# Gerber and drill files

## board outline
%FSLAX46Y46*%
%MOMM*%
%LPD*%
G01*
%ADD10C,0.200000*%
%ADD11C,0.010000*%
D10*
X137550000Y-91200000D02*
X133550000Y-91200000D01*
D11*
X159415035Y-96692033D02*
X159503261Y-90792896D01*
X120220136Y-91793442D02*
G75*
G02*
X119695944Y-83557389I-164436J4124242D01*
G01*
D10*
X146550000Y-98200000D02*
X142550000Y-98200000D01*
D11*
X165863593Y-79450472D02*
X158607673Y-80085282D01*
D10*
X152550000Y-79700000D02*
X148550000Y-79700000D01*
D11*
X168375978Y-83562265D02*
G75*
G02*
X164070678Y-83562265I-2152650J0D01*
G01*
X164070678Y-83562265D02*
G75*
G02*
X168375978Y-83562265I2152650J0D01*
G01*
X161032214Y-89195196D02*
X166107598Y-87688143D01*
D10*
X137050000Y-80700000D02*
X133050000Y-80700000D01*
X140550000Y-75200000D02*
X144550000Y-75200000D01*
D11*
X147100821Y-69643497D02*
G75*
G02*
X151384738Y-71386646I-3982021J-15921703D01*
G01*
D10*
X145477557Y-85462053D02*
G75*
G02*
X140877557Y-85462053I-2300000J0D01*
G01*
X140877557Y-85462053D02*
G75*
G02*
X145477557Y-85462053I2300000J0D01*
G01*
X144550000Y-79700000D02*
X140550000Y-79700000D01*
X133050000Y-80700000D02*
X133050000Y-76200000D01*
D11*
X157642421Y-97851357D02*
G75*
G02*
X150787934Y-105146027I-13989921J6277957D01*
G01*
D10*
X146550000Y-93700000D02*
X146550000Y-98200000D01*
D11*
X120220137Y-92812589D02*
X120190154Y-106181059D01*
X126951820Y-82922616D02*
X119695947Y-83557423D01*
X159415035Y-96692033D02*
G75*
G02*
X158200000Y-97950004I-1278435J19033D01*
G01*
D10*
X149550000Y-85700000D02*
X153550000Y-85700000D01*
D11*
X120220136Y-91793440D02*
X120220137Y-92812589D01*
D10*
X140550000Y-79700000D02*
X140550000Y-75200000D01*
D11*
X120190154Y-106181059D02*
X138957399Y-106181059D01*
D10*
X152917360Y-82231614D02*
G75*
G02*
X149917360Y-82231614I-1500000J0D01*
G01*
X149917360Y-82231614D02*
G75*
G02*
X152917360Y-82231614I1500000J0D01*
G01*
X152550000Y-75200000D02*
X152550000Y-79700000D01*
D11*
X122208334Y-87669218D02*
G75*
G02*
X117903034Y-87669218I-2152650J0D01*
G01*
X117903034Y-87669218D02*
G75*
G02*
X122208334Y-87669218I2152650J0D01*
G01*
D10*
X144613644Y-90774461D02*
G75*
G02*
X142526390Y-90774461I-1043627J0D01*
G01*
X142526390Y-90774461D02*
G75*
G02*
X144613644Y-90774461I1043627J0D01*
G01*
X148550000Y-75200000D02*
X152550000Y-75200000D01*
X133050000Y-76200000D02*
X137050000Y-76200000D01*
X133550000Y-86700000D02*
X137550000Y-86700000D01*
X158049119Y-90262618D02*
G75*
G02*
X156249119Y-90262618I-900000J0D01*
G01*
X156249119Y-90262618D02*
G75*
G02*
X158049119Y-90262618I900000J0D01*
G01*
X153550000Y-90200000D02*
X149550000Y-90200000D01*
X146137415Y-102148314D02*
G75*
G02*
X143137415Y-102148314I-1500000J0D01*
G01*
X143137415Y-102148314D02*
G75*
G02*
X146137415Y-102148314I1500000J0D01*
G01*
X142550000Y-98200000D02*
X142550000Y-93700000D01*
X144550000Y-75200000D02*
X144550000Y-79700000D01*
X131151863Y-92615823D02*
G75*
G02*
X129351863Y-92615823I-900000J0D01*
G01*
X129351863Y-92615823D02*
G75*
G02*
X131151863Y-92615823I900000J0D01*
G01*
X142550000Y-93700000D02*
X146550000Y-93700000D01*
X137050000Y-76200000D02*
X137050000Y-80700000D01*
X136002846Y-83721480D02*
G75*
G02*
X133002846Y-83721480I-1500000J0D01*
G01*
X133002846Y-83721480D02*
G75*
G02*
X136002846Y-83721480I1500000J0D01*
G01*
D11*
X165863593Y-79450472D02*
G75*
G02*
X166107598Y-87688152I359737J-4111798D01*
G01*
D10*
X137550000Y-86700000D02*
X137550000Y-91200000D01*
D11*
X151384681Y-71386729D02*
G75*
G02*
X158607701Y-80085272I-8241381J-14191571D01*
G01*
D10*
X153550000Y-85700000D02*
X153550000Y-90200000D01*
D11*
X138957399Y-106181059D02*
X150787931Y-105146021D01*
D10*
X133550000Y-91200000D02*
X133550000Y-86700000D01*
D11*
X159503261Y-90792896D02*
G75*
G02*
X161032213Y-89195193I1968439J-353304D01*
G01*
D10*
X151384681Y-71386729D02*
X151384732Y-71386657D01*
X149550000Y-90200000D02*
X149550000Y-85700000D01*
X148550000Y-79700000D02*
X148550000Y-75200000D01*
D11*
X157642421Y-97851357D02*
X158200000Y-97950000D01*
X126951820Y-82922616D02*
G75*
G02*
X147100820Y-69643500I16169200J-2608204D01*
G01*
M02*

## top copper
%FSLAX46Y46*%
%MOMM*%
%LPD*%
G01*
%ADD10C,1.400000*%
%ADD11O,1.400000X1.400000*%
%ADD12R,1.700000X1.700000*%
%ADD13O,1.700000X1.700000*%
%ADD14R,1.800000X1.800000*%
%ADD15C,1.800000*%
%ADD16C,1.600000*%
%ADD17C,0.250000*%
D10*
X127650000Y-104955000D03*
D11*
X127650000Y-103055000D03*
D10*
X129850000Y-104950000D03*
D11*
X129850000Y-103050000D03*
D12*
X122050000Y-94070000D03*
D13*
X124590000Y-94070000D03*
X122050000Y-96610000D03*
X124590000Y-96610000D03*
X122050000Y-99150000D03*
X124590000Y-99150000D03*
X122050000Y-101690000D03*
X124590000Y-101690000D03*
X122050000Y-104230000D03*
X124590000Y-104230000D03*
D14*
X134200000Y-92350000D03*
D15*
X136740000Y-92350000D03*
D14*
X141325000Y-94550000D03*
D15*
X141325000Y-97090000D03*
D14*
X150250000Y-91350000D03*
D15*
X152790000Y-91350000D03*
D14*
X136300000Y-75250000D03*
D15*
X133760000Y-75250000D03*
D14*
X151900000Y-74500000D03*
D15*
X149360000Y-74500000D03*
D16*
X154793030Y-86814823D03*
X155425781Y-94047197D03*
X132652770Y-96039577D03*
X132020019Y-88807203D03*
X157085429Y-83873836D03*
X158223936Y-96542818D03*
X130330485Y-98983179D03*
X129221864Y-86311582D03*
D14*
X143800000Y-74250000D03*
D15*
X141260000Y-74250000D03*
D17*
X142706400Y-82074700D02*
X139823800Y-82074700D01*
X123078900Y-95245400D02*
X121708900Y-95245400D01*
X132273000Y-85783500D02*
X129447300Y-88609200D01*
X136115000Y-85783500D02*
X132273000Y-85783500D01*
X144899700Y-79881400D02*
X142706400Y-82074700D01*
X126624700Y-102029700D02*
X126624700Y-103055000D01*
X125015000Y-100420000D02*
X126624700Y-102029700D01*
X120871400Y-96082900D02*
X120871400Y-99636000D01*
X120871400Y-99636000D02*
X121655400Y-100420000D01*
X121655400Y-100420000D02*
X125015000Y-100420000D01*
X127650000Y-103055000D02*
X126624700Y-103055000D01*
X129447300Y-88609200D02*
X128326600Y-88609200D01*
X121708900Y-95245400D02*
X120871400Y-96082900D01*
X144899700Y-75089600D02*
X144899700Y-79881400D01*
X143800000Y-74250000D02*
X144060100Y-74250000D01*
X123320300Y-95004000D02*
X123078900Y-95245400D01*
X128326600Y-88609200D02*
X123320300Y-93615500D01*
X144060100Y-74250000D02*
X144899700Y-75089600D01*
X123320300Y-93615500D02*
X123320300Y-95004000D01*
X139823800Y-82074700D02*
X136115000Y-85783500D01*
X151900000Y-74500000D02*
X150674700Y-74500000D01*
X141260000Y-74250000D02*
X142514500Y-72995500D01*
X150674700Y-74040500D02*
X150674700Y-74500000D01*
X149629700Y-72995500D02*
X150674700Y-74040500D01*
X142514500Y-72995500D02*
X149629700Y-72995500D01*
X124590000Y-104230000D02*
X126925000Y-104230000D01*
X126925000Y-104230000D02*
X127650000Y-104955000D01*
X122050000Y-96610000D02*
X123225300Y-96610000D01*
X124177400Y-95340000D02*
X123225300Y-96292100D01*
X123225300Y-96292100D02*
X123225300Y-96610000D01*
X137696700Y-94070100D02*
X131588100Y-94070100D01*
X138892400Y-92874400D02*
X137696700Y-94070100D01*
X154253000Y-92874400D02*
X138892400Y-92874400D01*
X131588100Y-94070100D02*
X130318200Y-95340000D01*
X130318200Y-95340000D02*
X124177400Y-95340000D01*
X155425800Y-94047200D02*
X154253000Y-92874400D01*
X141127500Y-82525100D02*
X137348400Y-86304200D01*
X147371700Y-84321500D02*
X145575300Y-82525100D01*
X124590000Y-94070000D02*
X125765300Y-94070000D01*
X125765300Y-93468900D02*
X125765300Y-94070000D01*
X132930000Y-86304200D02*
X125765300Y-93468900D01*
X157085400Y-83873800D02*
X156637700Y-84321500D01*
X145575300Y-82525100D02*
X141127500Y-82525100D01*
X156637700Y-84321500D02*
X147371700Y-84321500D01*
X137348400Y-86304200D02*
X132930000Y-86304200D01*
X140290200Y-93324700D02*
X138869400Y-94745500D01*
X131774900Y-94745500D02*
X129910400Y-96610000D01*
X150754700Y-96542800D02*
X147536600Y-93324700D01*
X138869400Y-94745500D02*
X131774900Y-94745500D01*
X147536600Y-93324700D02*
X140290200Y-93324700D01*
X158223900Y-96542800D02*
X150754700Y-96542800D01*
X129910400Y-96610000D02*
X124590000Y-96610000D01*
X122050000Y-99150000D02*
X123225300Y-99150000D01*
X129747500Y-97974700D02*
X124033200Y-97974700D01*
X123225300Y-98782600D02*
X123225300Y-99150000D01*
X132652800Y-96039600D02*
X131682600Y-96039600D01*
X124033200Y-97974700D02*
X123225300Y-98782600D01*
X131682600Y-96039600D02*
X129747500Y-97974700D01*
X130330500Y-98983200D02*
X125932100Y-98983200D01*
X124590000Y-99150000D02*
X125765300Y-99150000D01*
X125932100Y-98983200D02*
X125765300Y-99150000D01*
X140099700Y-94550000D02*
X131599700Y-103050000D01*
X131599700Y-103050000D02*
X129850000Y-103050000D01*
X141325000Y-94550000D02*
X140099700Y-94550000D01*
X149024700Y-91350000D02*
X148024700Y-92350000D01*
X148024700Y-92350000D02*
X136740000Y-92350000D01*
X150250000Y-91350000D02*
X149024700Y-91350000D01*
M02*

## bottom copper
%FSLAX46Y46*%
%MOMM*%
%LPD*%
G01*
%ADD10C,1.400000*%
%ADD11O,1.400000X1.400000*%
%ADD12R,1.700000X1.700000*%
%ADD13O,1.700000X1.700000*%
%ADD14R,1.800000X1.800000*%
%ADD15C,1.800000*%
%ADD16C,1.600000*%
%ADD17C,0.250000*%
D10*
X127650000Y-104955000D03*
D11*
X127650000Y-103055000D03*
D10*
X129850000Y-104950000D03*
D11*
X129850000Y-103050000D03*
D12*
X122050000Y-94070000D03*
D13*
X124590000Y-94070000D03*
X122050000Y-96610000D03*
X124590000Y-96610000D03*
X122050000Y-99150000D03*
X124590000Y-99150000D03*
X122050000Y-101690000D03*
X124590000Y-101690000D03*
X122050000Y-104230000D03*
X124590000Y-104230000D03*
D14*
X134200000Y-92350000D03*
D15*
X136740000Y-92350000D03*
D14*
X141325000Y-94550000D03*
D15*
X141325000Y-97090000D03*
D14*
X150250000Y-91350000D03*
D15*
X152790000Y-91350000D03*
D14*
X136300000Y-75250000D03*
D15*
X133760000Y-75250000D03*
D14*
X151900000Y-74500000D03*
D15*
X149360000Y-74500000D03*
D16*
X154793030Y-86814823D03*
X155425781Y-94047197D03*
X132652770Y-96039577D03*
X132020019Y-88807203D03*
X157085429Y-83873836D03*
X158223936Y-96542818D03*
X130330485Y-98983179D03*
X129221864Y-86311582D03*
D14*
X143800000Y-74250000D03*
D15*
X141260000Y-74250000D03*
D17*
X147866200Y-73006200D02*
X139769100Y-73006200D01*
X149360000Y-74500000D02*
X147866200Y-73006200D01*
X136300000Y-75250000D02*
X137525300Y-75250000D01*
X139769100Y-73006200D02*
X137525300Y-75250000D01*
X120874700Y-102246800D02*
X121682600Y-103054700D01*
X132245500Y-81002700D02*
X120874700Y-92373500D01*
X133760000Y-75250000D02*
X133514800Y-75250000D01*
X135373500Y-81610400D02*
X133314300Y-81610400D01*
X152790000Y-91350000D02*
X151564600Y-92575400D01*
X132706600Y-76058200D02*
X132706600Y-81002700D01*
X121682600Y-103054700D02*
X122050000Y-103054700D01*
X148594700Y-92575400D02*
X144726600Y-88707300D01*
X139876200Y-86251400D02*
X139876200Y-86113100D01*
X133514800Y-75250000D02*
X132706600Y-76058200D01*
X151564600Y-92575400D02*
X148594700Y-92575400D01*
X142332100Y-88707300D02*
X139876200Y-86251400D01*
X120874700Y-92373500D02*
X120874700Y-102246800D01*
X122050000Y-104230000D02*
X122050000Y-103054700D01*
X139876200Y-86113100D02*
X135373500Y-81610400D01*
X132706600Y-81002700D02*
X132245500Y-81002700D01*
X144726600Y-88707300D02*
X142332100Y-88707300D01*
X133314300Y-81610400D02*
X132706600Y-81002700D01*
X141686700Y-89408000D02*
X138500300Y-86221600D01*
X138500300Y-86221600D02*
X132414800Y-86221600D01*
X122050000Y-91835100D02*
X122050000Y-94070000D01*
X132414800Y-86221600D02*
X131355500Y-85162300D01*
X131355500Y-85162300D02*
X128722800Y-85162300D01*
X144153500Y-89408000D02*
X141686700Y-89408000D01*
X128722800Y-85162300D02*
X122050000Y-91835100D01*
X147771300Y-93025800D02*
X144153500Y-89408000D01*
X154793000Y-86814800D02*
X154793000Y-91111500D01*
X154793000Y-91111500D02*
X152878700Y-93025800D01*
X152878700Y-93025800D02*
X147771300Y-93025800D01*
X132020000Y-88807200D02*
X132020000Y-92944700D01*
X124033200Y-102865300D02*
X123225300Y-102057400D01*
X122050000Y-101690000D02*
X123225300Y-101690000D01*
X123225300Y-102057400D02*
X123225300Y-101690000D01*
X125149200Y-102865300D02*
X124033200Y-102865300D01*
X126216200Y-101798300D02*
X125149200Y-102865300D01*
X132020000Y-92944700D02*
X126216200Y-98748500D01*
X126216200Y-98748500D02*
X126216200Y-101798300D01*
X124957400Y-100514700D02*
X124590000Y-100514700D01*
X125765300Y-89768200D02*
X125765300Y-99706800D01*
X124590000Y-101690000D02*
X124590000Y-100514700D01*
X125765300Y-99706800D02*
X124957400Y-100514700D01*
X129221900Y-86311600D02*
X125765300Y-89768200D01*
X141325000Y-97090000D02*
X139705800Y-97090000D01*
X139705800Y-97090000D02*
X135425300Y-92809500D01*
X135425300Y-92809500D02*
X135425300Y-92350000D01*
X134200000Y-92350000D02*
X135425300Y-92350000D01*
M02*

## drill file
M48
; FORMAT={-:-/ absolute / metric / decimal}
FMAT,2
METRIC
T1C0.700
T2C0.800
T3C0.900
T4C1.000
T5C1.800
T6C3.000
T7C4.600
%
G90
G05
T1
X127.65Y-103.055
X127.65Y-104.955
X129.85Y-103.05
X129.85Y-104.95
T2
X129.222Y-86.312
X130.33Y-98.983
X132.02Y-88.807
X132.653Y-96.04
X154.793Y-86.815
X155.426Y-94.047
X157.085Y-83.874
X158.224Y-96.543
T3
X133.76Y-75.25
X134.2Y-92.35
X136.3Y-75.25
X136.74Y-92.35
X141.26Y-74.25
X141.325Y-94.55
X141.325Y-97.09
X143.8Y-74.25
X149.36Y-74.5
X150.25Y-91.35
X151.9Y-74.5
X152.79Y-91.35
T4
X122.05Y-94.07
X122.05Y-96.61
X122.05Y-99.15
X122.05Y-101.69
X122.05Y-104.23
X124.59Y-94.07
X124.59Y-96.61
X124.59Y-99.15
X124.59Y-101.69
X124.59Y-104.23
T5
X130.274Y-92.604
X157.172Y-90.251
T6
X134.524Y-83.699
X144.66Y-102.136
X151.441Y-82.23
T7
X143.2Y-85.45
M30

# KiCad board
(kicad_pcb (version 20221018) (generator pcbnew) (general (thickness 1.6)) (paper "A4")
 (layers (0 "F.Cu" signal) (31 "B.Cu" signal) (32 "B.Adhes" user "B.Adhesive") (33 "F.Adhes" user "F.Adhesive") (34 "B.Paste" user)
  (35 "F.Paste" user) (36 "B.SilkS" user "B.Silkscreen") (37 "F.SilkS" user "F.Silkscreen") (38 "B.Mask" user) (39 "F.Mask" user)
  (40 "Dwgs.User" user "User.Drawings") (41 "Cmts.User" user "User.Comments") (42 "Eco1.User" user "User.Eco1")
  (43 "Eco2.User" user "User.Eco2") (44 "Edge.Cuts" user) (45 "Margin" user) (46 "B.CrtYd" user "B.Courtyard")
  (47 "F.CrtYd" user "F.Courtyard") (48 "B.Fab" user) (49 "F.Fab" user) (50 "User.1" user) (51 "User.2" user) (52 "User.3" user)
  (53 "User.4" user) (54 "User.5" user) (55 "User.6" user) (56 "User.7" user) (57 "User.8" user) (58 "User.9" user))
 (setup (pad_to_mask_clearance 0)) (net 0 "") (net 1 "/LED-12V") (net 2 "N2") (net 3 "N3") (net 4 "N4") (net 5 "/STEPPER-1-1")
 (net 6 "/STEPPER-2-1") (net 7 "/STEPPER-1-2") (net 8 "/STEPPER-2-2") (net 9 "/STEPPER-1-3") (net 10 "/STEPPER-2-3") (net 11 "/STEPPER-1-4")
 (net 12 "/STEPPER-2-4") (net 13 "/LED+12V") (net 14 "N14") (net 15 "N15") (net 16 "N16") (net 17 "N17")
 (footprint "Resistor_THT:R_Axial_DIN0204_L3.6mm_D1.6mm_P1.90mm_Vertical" (layer "F.Cu") (at 127.65 104.955 90)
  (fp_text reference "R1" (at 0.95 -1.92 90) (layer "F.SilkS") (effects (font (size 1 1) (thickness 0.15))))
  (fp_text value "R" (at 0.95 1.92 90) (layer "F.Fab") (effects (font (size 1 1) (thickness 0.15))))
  (pad "1" thru_hole circle (at 0 0 90) (size 1.4 1.4) (drill 0.7) (layers "*.Cu" "*.Mask") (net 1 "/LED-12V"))
  (pad "2" thru_hole oval (at 1.9 0 90) (size 1.4 1.4) (drill 0.7) (layers "*.Cu" "*.Mask") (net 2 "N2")))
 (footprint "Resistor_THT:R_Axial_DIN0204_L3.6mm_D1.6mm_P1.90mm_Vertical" (layer "F.Cu") (at 129.85 104.95 90)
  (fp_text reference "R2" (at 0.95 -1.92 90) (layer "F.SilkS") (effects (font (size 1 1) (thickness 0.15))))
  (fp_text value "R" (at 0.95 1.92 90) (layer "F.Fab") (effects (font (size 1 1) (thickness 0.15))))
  (pad "1" thru_hole circle (at 0 0 90) (size 1.4 1.4) (drill 0.7) (layers "*.Cu" "*.Mask") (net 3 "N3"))
  (pad "2" thru_hole oval (at 1.9 0 90) (size 1.4 1.4) (drill 0.7) (layers "*.Cu" "*.Mask") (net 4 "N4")))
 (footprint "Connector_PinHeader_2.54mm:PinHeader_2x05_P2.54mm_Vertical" (layer "F.Cu") (at 122.05 94.07)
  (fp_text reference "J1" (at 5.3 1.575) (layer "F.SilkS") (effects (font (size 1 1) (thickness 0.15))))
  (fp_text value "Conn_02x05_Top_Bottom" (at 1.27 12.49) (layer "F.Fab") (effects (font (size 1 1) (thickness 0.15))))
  (pad "1" thru_hole rect (at 0 0) (size 1.7 1.7) (drill 1) (layers "*.Cu" "*.Mask") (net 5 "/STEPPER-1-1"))
  (pad "2" thru_hole oval (at 2.54 0) (size 1.7 1.7) (drill 1) (layers "*.Cu" "*.Mask") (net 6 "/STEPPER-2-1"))
  (pad "3" thru_hole oval (at 0 2.54) (size 1.7 1.7) (drill 1) (layers "*.Cu" "*.Mask") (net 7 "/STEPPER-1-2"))
  (pad "4" thru_hole oval (at 2.54 2.54) (size 1.7 1.7) (drill 1) (layers "*.Cu" "*.Mask") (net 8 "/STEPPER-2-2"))
  (pad "5" thru_hole oval (at 0 5.08) (size 1.7 1.7) (drill 1) (layers "*.Cu" "*.Mask") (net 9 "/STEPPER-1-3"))
  (pad "6" thru_hole oval (at 2.54 5.08) (size 1.7 1.7) (drill 1) (layers "*.Cu" "*.Mask") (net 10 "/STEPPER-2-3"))
  (pad "7" thru_hole oval (at 0 7.62) (size 1.7 1.7) (drill 1) (layers "*.Cu" "*.Mask") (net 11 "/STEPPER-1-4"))
  (pad "8" thru_hole oval (at 2.54 7.62) (size 1.7 1.7) (drill 1) (layers "*.Cu" "*.Mask") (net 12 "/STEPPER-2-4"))
  (pad "9" thru_hole oval (at 0 10.16) (size 1.7 1.7) (drill 1) (layers "*.Cu" "*.Mask") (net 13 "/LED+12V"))
  (pad "10" thru_hole oval (at 2.54 10.16) (size 1.7 1.7) (drill 1) (layers "*.Cu" "*.Mask") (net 1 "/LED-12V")))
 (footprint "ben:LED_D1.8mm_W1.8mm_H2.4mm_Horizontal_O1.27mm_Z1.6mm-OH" (layer "B.Cu") (at 134.2 92.35)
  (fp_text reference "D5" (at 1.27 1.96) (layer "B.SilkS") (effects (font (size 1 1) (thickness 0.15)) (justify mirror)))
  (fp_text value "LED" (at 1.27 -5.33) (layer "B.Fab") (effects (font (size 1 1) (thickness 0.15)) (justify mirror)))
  (pad "1" thru_hole rect (at 0 0) (size 1.8 1.8) (drill 0.9) (layers "*.Cu" "*.Mask") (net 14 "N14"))
  (pad "2" thru_hole circle (at 2.54 0) (size 1.8 1.8) (drill 0.9) (layers "*.Cu" "*.Mask") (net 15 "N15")))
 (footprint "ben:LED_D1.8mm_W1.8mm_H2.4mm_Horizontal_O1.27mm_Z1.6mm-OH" (layer "B.Cu") (at 141.325 94.55 -90)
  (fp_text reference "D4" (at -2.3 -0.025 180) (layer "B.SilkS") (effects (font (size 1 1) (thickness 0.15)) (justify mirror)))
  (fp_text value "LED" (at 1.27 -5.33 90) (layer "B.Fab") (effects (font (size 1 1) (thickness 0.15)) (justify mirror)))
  (pad "1" thru_hole rect (at 0 0 270) (size 1.8 1.8) (drill 0.9) (layers "*.Cu" "*.Mask") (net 4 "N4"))
  (pad "2" thru_hole circle (at 2.54 0 270) (size 1.8 1.8) (drill 0.9) (layers "*.Cu" "*.Mask") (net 14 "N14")))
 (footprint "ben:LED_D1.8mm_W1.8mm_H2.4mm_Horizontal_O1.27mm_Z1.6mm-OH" (layer "B.Cu") (at 150.25 91.35)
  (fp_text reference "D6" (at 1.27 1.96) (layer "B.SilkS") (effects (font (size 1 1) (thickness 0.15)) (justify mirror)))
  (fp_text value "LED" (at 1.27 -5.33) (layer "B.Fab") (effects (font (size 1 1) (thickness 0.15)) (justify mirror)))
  (pad "1" thru_hole rect (at 0 0) (size 1.8 1.8) (drill 0.9) (layers "*.Cu" "*.Mask") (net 15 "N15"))
  (pad "2" thru_hole circle (at 2.54 0) (size 1.8 1.8) (drill 0.9) (layers "*.Cu" "*.Mask") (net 13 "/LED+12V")))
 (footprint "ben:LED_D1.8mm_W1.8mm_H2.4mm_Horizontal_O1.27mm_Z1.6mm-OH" (layer "B.Cu") (at 136.3 75.25 180)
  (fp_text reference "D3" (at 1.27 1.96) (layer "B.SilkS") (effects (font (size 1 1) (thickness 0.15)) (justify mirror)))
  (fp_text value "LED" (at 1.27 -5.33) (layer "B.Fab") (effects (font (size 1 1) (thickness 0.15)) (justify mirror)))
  (pad "1" thru_hole rect (at 0 0 180) (size 1.8 1.8) (drill 0.9) (layers "*.Cu" "*.Mask") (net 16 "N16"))
  (pad "2" thru_hole circle (at 2.54 0 180) (size 1.8 1.8) (drill 0.9) (layers "*.Cu" "*.Mask") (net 13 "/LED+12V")))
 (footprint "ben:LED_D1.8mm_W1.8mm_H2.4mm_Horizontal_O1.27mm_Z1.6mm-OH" (layer "B.Cu") (at 151.9 74.5 180)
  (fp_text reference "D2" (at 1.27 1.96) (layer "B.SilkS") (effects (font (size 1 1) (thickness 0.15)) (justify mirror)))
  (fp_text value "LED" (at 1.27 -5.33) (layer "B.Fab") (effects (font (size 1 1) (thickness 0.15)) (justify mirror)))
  (pad "1" thru_hole rect (at 0 0 180) (size 1.8 1.8) (drill 0.9) (layers "*.Cu" "*.Mask") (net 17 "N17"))
  (pad "2" thru_hole circle (at 2.54 0 180) (size 1.8 1.8) (drill 0.9) (layers "*.Cu" "*.Mask") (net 16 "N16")))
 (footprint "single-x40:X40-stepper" (layer "B.Cu") (at 143.7229 91.4272 -175)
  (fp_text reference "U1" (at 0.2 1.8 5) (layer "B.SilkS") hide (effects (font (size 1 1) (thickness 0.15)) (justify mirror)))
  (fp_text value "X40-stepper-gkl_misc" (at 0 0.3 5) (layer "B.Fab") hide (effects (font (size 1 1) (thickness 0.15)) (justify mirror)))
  (pad "" np_thru_hole circle (at -13.5 0 185) (size 1.8 1.8) (drill 1.8) (layers "*.Cu" "*.Mask"))
  (pad "" np_thru_hole circle (at -8.49 8.49 185) (size 3 3) (drill 3) (layers "*.Cu" "*.Mask"))
  (pad "" np_thru_hole circle (at 0 -10.75 185) (size 3 3) (drill 3) (layers "*.Cu" "*.Mask"))
  (pad "" np_thru_hole circle (at 0 6 185) (size 4.6 4.6) (drill 4.6) (layers "*.Cu" "*.Mask"))
  (pad "" np_thru_hole circle (at 8.49 8.5 185) (size 3 3) (drill 3) (layers "*.Cu" "*.Mask"))
  (pad "" np_thru_hole circle (at 13.5 0 185) (size 1.8 1.8) (drill 1.8) (layers "*.Cu" "*.Mask"))
  (pad "1" thru_hole circle (at -11.43 3.63 185) (size 1.6 1.6) (drill 0.8) (layers "*.Cu" "*.Mask") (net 5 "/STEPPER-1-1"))
  (pad "2" thru_hole circle (at -11.43 -3.63 185) (size 1.6 1.6) (drill 0.8) (layers "*.Cu" "*.Mask") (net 7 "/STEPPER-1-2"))
  (pad "3" thru_hole circle (at 11.43 -3.63 185) (size 1.6 1.6) (drill 0.8) (layers "*.Cu" "*.Mask") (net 9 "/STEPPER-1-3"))
  (pad "4" thru_hole circle (at 11.43 3.63 185) (size 1.6 1.6) (drill 0.8) (layers "*.Cu" "*.Mask") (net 11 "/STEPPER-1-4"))
  (pad "5" thru_hole circle (at -13.97 6.36 185) (size 1.6 1.6) (drill 0.8) (layers "*.Cu" "*.Mask") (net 6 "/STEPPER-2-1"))
  (pad "6" thru_hole circle (at -14 -6.36 185) (size 1.6 1.6) (drill 0.8) (layers "*.Cu" "*.Mask") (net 8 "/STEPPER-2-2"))
  (pad "7" thru_hole circle (at 14 -6.36 185) (size 1.6 1.6) (drill 0.8) (layers "*.Cu" "*.Mask") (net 10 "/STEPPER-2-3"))
  (pad "8" thru_hole circle (at 14 6.36 185) (size 1.6 1.6) (drill 0.8) (layers "*.Cu" "*.Mask") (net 12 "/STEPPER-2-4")))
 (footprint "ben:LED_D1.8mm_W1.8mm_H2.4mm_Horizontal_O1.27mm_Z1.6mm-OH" (layer "B.Cu") (at 143.8 74.25 180)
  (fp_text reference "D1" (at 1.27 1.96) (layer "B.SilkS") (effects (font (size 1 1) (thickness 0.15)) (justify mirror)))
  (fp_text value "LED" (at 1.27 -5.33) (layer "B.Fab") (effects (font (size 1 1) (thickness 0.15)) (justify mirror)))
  (pad "1" thru_hole rect (at 0 0 180) (size 1.8 1.8) (drill 0.9) (layers "*.Cu" "*.Mask") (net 2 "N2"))
  (pad "2" thru_hole circle (at 2.54 0 180) (size 1.8 1.8) (drill 0.9) (layers "*.Cu" "*.Mask") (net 17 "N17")))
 (gr_line (start 137.55 91.2) (end 133.55 91.2) (stroke (width 0.2) (type solid)) (layer "Edge.Cuts"))
 (gr_line (start 159.415035 96.692033) (end 159.503261 90.792896) (stroke (width 0.01) (type solid)) (layer "Edge.Cuts"))
 (gr_arc (start 120.220136 91.793442) (mid 115.936516 87.931386) (end 119.695947 83.557423) (stroke (width 0.01) (type solid))
  (layer "Edge.Cuts"))
 (gr_line (start 146.55 98.2) (end 142.55 98.2) (stroke (width 0.2) (type solid)) (layer "Edge.Cuts"))
 (gr_line (start 165.863593 79.450472) (end 158.607673 80.085282) (stroke (width 0.01) (type solid)) (layer "Edge.Cuts"))
 (gr_line (start 152.55 79.7) (end 148.55 79.7) (stroke (width 0.2) (type solid)) (layer "Edge.Cuts"))
 (gr_circle (center 166.223328 83.562265) (end 168.375978 83.562265) (stroke (width 0.01) (type solid)) (fill none) (layer "Edge.Cuts"))
 (gr_line (start 161.032214 89.195196) (end 166.107598 87.688143) (stroke (width 0.01) (type solid)) (layer "Edge.Cuts"))
 (gr_line (start 137.05 80.7) (end 133.05 80.7) (stroke (width 0.2) (type solid)) (layer "Edge.Cuts"))
 (gr_line (start 140.55 75.2) (end 144.55 75.2) (stroke (width 0.2) (type solid)) (layer "Edge.Cuts"))
 (gr_arc (start 147.100821 69.643497) (mid 149.304488 70.363418) (end 151.384732 71.386657) (stroke (width 0.01) (type solid))
  (layer "Edge.Cuts"))
 (gr_circle (center 143.177557 85.462053) (end 140.877557 85.462053) (stroke (width 0.2) (type solid)) (fill none) (layer "Edge.Cuts"))
 (gr_line (start 144.55 79.7) (end 140.55 79.7) (stroke (width 0.2) (type solid)) (layer "Edge.Cuts"))
 (gr_line (start 133.05 80.7) (end 133.05 76.2) (stroke (width 0.2) (type solid)) (layer "Edge.Cuts"))
 (gr_arc (start 157.642421 97.851357) (mid 154.827166 102.07375) (end 150.787931 105.146021) (stroke (width 0.01) (type solid))
  (layer "Edge.Cuts"))
 (gr_line (start 146.55 93.7) (end 146.55 98.2) (stroke (width 0.2) (type solid)) (layer "Edge.Cuts"))
 (gr_line (start 120.220137 92.812589) (end 120.190154 106.181059) (stroke (width 0.01) (type solid)) (layer "Edge.Cuts"))
 (gr_line (start 126.95182 82.922616) (end 119.695947 83.557423) (stroke (width 0.01) (type solid)) (layer "Edge.Cuts"))
 (gr_arc (start 159.415035 96.692033) (mid 159.056246 97.561256) (end 158.2 97.95) (stroke (width 0.01) (type solid)) (layer "Edge.Cuts"))
 (gr_line (start 149.55 85.7) (end 153.55 85.7) (stroke (width 0.2) (type solid)) (layer "Edge.Cuts"))
 (gr_line (start 120.220136 91.79344) (end 120.220137 92.812589) (stroke (width 0.01) (type solid)) (layer "Edge.Cuts"))
 (gr_line (start 140.55 79.7) (end 140.55 75.2) (stroke (width 0.2) (type solid)) (layer "Edge.Cuts"))
 (gr_line (start 120.190154 106.181059) (end 138.957399 106.181059) (stroke (width 0.01) (type solid)) (layer "Edge.Cuts"))
 (gr_circle (center 151.41736 82.231614) (end 149.91736 82.231614) (stroke (width 0.2) (type solid)) (fill none) (layer "Edge.Cuts"))
 (gr_line (start 152.55 75.2) (end 152.55 79.7) (stroke (width 0.2) (type solid)) (layer "Edge.Cuts"))
 (gr_circle (center 120.055684 87.669218) (end 122.208334 87.669218) (stroke (width 0.01) (type solid)) (fill none) (layer "Edge.Cuts"))
 (gr_circle (center 143.570017 90.774461) (end 142.52639 90.774461) (stroke (width 0.2) (type solid)) (fill none) (layer "Edge.Cuts"))
 (gr_line (start 148.55 75.2) (end 152.55 75.2) (stroke (width 0.2) (type solid)) (layer "Edge.Cuts"))
 (gr_line (start 133.05 76.2) (end 137.05 76.2) (stroke (width 0.2) (type solid)) (layer "Edge.Cuts"))
 (gr_line (start 133.55 86.7) (end 137.55 86.7) (stroke (width 0.2) (type solid)) (layer "Edge.Cuts"))
 (gr_circle (center 157.149119 90.262618) (end 156.249119 90.262618) (stroke (width 0.2) (type solid)) (fill none) (layer "Edge.Cuts"))
 (gr_line (start 153.55 90.2) (end 149.55 90.2) (stroke (width 0.2) (type solid)) (layer "Edge.Cuts"))
 (gr_circle (center 144.637415 102.148314) (end 143.137415 102.148314) (stroke (width 0.2) (type solid)) (fill none) (layer "Edge.Cuts"))
 (gr_line (start 142.55 98.2) (end 142.55 93.7) (stroke (width 0.2) (type solid)) (layer "Edge.Cuts"))
 (gr_line (start 144.55 75.2) (end 144.55 79.7) (stroke (width 0.2) (type solid)) (layer "Edge.Cuts"))
 (gr_circle (center 130.251863 92.615823) (end 129.351863 92.615823) (stroke (width 0.2) (type solid)) (fill none) (layer "Edge.Cuts"))
 (gr_line (start 142.55 93.7) (end 146.55 93.7) (stroke (width 0.2) (type solid)) (layer "Edge.Cuts"))
 (gr_line (start 137.05 76.2) (end 137.05 80.7) (stroke (width 0.2) (type solid)) (layer "Edge.Cuts"))
 (gr_circle (center 134.502846 83.72148) (end 133.002846 83.72148) (stroke (width 0.2) (type solid)) (fill none) (layer "Edge.Cuts"))
 (gr_arc (start 165.863593 79.450472) (mid 170.349018 83.44006) (end 166.107598 87.688143) (stroke (width 0.01) (type solid))
  (layer "Edge.Cuts"))
 (gr_line (start 137.55 86.7) (end 137.55 91.2) (stroke (width 0.2) (type solid)) (layer "Edge.Cuts"))
 (gr_arc (start 151.384681 71.386729) (mid 155.768943 75.094326) (end 158.607673 80.085282) (stroke (width 0.01) (type solid))
  (layer "Edge.Cuts"))
 (gr_line (start 153.55 85.7) (end 153.55 90.2) (stroke (width 0.2) (type solid)) (layer "Edge.Cuts"))
 (gr_line (start 138.957399 106.181059) (end 150.787931 105.146021) (stroke (width 0.01) (type solid)) (layer "Edge.Cuts"))
 (gr_line (start 133.55 91.2) (end 133.55 86.7) (stroke (width 0.2) (type solid)) (layer "Edge.Cuts"))
 (gr_arc (start 159.503261 90.792896) (mid 160.026816 89.76349) (end 161.032214 89.195196) (stroke (width 0.01) (type solid))
  (layer "Edge.Cuts"))
 (gr_line (start 151.384681 71.386729) (end 151.384732 71.386657) (stroke (width 0.2) (type solid)) (layer "Edge.Cuts"))
 (gr_line (start 149.55 90.2) (end 149.55 85.7) (stroke (width 0.2) (type solid)) (layer "Edge.Cuts"))
 (gr_line (start 148.55 79.7) (end 148.55 75.2) (stroke (width 0.2) (type solid)) (layer "Edge.Cuts"))
 (gr_line (start 157.642421 97.851357) (end 158.2 97.95) (stroke (width 0.01) (type solid)) (layer "Edge.Cuts"))
 (gr_arc (start 126.95182 82.922616) (mid 134.108302 71.855416) (end 147.100821 69.643497) (stroke (width 0.01) (type solid))
  (layer "Edge.Cuts"))
 (segment (start 142.7064 82.0747) (end 139.8238 82.0747) (width 0.25) (layer "F.Cu") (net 2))
 (segment (start 123.0789 95.2454) (end 121.7089 95.2454) (width 0.25) (layer "F.Cu") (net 2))
 (segment (start 132.273 85.7835) (end 129.4473 88.6092) (width 0.25) (layer "F.Cu") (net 2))
 (segment (start 136.115 85.7835) (end 132.273 85.7835) (width 0.25) (layer "F.Cu") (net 2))
 (segment (start 144.8997 79.8814) (end 142.7064 82.0747) (width 0.25) (layer "F.Cu") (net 2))
 (segment (start 126.6247 102.0297) (end 126.6247 103.055) (width 0.25) (layer "F.Cu") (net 2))
 (segment (start 125.015 100.42) (end 126.6247 102.0297) (width 0.25) (layer "F.Cu") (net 2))
 (segment (start 120.8714 96.0829) (end 120.8714 99.636) (width 0.25) (layer "F.Cu") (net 2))
 (segment (start 120.8714 99.636) (end 121.6554 100.42) (width 0.25) (layer "F.Cu") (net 2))
 (segment (start 121.6554 100.42) (end 125.015 100.42) (width 0.25) (layer "F.Cu") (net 2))
 (segment (start 127.65 103.055) (end 126.6247 103.055) (width 0.25) (layer "F.Cu") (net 2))
 (segment (start 129.4473 88.6092) (end 128.3266 88.6092) (width 0.25) (layer "F.Cu") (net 2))
 (segment (start 121.7089 95.2454) (end 120.8714 96.0829) (width 0.25) (layer "F.Cu") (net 2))
 (segment (start 144.8997 75.0896) (end 144.8997 79.8814) (width 0.25) (layer "F.Cu") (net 2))
 (segment (start 143.8 74.25) (end 144.0601 74.25) (width 0.25) (layer "F.Cu") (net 2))
 (segment (start 123.3203 95.004) (end 123.0789 95.2454) (width 0.25) (layer "F.Cu") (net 2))
 (segment (start 128.3266 88.6092) (end 123.3203 93.6155) (width 0.25) (layer "F.Cu") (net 2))
 (segment (start 144.0601 74.25) (end 144.8997 75.0896) (width 0.25) (layer "F.Cu") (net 2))
 (segment (start 123.3203 93.6155) (end 123.3203 95.004) (width 0.25) (layer "F.Cu") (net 2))
 (segment (start 139.8238 82.0747) (end 136.115 85.7835) (width 0.25) (layer "F.Cu") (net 2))
 (segment (start 151.9 74.5) (end 150.6747 74.5) (width 0.25) (layer "F.Cu") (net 17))
 (segment (start 141.26 74.25) (end 142.5145 72.9955) (width 0.25) (layer "F.Cu") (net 17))
 (segment (start 150.6747 74.0405) (end 150.6747 74.5) (width 0.25) (layer "F.Cu") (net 17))
 (segment (start 149.6297 72.9955) (end 150.6747 74.0405) (width 0.25) (layer "F.Cu") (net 17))
 (segment (start 142.5145 72.9955) (end 149.6297 72.9955) (width 0.25) (layer "F.Cu") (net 17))
 (segment (start 147.8662 73.0062) (end 139.7691 73.0062) (width 0.25) (layer "B.Cu") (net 16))
 (segment (start 149.36 74.5) (end 147.8662 73.0062) (width 0.25) (layer "B.Cu") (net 16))
 (segment (start 136.3 75.25) (end 137.5253 75.25) (width 0.25) (layer "B.Cu") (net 16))
 (segment (start 139.7691 73.0062) (end 137.5253 75.25) (width 0.25) (layer "B.Cu") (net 16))
 (segment (start 120.8747 102.2468) (end 121.6826 103.0547) (width 0.25) (layer "B.Cu") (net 13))
 (segment (start 132.2455 81.0027) (end 120.8747 92.3735) (width 0.25) (layer "B.Cu") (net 13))
 (segment (start 133.76 75.25) (end 133.5148 75.25) (width 0.25) (layer "B.Cu") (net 13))
 (segment (start 135.3735 81.6104) (end 133.3143 81.6104) (width 0.25) (layer "B.Cu") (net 13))
 (segment (start 152.79 91.35) (end 151.5646 92.5754) (width 0.25) (layer "B.Cu") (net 13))
 (segment (start 132.7066 76.0582) (end 132.7066 81.0027) (width 0.25) (layer "B.Cu") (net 13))
 (segment (start 121.6826 103.0547) (end 122.05 103.0547) (width 0.25) (layer "B.Cu") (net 13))
 (segment (start 148.5947 92.5754) (end 144.7266 88.7073) (width 0.25) (layer "B.Cu") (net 13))
 (segment (start 139.8762 86.2514) (end 139.8762 86.1131) (width 0.25) (layer "B.Cu") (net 13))
 (segment (start 133.5148 75.25) (end 132.7066 76.0582) (width 0.25) (layer "B.Cu") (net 13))
 (segment (start 151.5646 92.5754) (end 148.5947 92.5754) (width 0.25) (layer "B.Cu") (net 13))
 (segment (start 142.3321 88.7073) (end 139.8762 86.2514) (width 0.25) (layer "B.Cu") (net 13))
 (segment (start 120.8747 92.3735) (end 120.8747 102.2468) (width 0.25) (layer "B.Cu") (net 13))
 (segment (start 122.05 104.23) (end 122.05 103.0547) (width 0.25) (layer "B.Cu") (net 13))
 (segment (start 139.8762 86.1131) (end 135.3735 81.6104) (width 0.25) (layer "B.Cu") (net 13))
 (segment (start 132.7066 81.0027) (end 132.2455 81.0027) (width 0.25) (layer "B.Cu") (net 13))
 (segment (start 144.7266 88.7073) (end 142.3321 88.7073) (width 0.25) (layer "B.Cu") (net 13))
 (segment (start 133.3143 81.6104) (end 132.7066 81.0027) (width 0.25) (layer "B.Cu") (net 13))
 (segment (start 124.59 104.23) (end 126.925 104.23) (width 0.25) (layer "F.Cu") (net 1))
 (segment (start 126.925 104.23) (end 127.65 104.955) (width 0.25) (layer "F.Cu") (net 1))
 (segment (start 141.6867 89.408) (end 138.5003 86.2216) (width 0.25) (layer "B.Cu") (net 5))
 (segment (start 138.5003 86.2216) (end 132.4148 86.2216) (width 0.25) (layer "B.Cu") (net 5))
 (segment (start 122.05 91.8351) (end 122.05 94.07) (width 0.25) (layer "B.Cu") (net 5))
 (segment (start 132.4148 86.2216) (end 131.3555 85.1623) (width 0.25) (layer "B.Cu") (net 5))
 (segment (start 131.3555 85.1623) (end 128.7228 85.1623) (width 0.25) (layer "B.Cu") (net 5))
 (segment (start 144.1535 89.408) (end 141.6867 89.408) (width 0.25) (layer "B.Cu") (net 5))
 (segment (start 128.7228 85.1623) (end 122.05 91.8351) (width 0.25) (layer "B.Cu") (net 5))
 (segment (start 147.7713 93.0258) (end 144.1535 89.408) (width 0.25) (layer "B.Cu") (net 5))
 (segment (start 154.793 86.8148) (end 154.793 91.1115) (width 0.25) (layer "B.Cu") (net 5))
 (segment (start 154.793 91.1115) (end 152.8787 93.0258) (width 0.25) (layer "B.Cu") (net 5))
 (segment (start 152.8787 93.0258) (end 147.7713 93.0258) (width 0.25) (layer "B.Cu") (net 5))
 (segment (start 122.05 96.61) (end 123.2253 96.61) (width 0.25) (layer "F.Cu") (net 7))
 (segment (start 124.1774 95.34) (end 123.2253 96.2921) (width 0.25) (layer "F.Cu") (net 7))
 (segment (start 123.2253 96.2921) (end 123.2253 96.61) (width 0.25) (layer "F.Cu") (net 7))
 (segment (start 137.6967 94.0701) (end 131.5881 94.0701) (width 0.25) (layer "F.Cu") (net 7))
 (segment (start 138.8924 92.8744) (end 137.6967 94.0701) (width 0.25) (layer "F.Cu") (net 7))
 (segment (start 154.253 92.8744) (end 138.8924 92.8744) (width 0.25) (layer "F.Cu") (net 7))
 (segment (start 131.5881 94.0701) (end 130.3182 95.34) (width 0.25) (layer "F.Cu") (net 7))
 (segment (start 130.3182 95.34) (end 124.1774 95.34) (width 0.25) (layer "F.Cu") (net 7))
 (segment (start 155.4258 94.0472) (end 154.253 92.8744) (width 0.25) (layer "F.Cu") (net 7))
 (segment (start 141.1275 82.5251) (end 137.3484 86.3042) (width 0.25) (layer "F.Cu") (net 6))
 (segment (start 147.3717 84.3215) (end 145.5753 82.5251) (width 0.25) (layer "F.Cu") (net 6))
 (segment (start 124.59 94.07) (end 125.7653 94.07) (width 0.25) (layer "F.Cu") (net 6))
 (segment (start 125.7653 93.4689) (end 125.7653 94.07) (width 0.25) (layer "F.Cu") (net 6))
 (segment (start 132.93 86.3042) (end 125.7653 93.4689) (width 0.25) (layer "F.Cu") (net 6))
 (segment (start 157.0854 83.8738) (end 156.6377 84.3215) (width 0.25) (layer "F.Cu") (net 6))
 (segment (start 145.5753 82.5251) (end 141.1275 82.5251) (width 0.25) (layer "F.Cu") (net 6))
 (segment (start 156.6377 84.3215) (end 147.3717 84.3215) (width 0.25) (layer "F.Cu") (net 6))
 (segment (start 137.3484 86.3042) (end 132.93 86.3042) (width 0.25) (layer "F.Cu") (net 6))
 (segment (start 140.2902 93.3247) (end 138.8694 94.7455) (width 0.25) (layer "F.Cu") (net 8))
 (segment (start 131.7749 94.7455) (end 129.9104 96.61) (width 0.25) (layer "F.Cu") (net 8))
 (segment (start 150.7547 96.5428) (end 147.5366 93.3247) (width 0.25) (layer "F.Cu") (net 8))
 (segment (start 138.8694 94.7455) (end 131.7749 94.7455) (width 0.25) (layer "F.Cu") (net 8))
 (segment (start 147.5366 93.3247) (end 140.2902 93.3247) (width 0.25) (layer "F.Cu") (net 8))
 (segment (start 158.2239 96.5428) (end 150.7547 96.5428) (width 0.25) (layer "F.Cu") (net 8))
 (segment (start 129.9104 96.61) (end 124.59 96.61) (width 0.25) (layer "F.Cu") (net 8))
 (segment (start 132.02 88.8072) (end 132.02 92.9447) (width 0.25) (layer "B.Cu") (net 11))
 (segment (start 124.0332 102.8653) (end 123.2253 102.0574) (width 0.25) (layer "B.Cu") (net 11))
 (segment (start 122.05 101.69) (end 123.2253 101.69) (width 0.25) (layer "B.Cu") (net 11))
 (segment (start 123.2253 102.0574) (end 123.2253 101.69) (width 0.25) (layer "B.Cu") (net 11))
 (segment (start 125.1492 102.8653) (end 124.0332 102.8653) (width 0.25) (layer "B.Cu") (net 11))
 (segment (start 126.2162 101.7983) (end 125.1492 102.8653) (width 0.25) (layer "B.Cu") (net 11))
 (segment (start 132.02 92.9447) (end 126.2162 98.7485) (width 0.25) (layer "B.Cu") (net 11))
 (segment (start 126.2162 98.7485) (end 126.2162 101.7983) (width 0.25) (layer "B.Cu") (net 11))
 (segment (start 122.05 99.15) (end 123.2253 99.15) (width 0.25) (layer "F.Cu") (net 9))
 (segment (start 129.7475 97.9747) (end 124.0332 97.9747) (width 0.25) (layer "F.Cu") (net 9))
 (segment (start 123.2253 98.7826) (end 123.2253 99.15) (width 0.25) (layer "F.Cu") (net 9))
 (segment (start 132.6528 96.0396) (end 131.6826 96.0396) (width 0.25) (layer "F.Cu") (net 9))
 (segment (start 124.0332 97.9747) (end 123.2253 98.7826) (width 0.25) (layer "F.Cu") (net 9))
 (segment (start 131.6826 96.0396) (end 129.7475 97.9747) (width 0.25) (layer "F.Cu") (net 9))
 (segment (start 124.9574 100.5147) (end 124.59 100.5147) (width 0.25) (layer "B.Cu") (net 12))
 (segment (start 125.7653 89.7682) (end 125.7653 99.7068) (width 0.25) (layer "B.Cu") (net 12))
 (segment (start 124.59 101.69) (end 124.59 100.5147) (width 0.25) (layer "B.Cu") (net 12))
 (segment (start 125.7653 99.7068) (end 124.9574 100.5147) (width 0.25) (layer "B.Cu") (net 12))
 (segment (start 129.2219 86.3116) (end 125.7653 89.7682) (width 0.25) (layer "B.Cu") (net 12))
 (segment (start 130.3305 98.9832) (end 125.9321 98.9832) (width 0.25) (layer "F.Cu") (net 10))
 (segment (start 124.59 99.15) (end 125.7653 99.15) (width 0.25) (layer "F.Cu") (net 10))
 (segment (start 125.9321 98.9832) (end 125.7653 99.15) (width 0.25) (layer "F.Cu") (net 10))
 (segment (start 140.0997 94.55) (end 131.5997 103.05) (width 0.25) (layer "F.Cu") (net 4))
 (segment (start 131.5997 103.05) (end 129.85 103.05) (width 0.25) (layer "F.Cu") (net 4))
 (segment (start 141.325 94.55) (end 140.0997 94.55) (width 0.25) (layer "F.Cu") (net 4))
 (segment (start 141.325 97.09) (end 139.7058 97.09) (width 0.25) (layer "B.Cu") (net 14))
 (segment (start 139.7058 97.09) (end 135.4253 92.8095) (width 0.25) (layer "B.Cu") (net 14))
 (segment (start 135.4253 92.8095) (end 135.4253 92.35) (width 0.25) (layer "B.Cu") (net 14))
 (segment (start 134.2 92.35) (end 135.4253 92.35) (width 0.25) (layer "B.Cu") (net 14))
 (segment (start 149.0247 91.35) (end 148.0247 92.35) (width 0.25) (layer "F.Cu") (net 15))
 (segment (start 148.0247 92.35) (end 136.74 92.35) (width 0.25) (layer "F.Cu") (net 15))
 (segment (start 150.25 91.35) (end 149.0247 91.35) (width 0.25) (layer "F.Cu") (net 15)))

